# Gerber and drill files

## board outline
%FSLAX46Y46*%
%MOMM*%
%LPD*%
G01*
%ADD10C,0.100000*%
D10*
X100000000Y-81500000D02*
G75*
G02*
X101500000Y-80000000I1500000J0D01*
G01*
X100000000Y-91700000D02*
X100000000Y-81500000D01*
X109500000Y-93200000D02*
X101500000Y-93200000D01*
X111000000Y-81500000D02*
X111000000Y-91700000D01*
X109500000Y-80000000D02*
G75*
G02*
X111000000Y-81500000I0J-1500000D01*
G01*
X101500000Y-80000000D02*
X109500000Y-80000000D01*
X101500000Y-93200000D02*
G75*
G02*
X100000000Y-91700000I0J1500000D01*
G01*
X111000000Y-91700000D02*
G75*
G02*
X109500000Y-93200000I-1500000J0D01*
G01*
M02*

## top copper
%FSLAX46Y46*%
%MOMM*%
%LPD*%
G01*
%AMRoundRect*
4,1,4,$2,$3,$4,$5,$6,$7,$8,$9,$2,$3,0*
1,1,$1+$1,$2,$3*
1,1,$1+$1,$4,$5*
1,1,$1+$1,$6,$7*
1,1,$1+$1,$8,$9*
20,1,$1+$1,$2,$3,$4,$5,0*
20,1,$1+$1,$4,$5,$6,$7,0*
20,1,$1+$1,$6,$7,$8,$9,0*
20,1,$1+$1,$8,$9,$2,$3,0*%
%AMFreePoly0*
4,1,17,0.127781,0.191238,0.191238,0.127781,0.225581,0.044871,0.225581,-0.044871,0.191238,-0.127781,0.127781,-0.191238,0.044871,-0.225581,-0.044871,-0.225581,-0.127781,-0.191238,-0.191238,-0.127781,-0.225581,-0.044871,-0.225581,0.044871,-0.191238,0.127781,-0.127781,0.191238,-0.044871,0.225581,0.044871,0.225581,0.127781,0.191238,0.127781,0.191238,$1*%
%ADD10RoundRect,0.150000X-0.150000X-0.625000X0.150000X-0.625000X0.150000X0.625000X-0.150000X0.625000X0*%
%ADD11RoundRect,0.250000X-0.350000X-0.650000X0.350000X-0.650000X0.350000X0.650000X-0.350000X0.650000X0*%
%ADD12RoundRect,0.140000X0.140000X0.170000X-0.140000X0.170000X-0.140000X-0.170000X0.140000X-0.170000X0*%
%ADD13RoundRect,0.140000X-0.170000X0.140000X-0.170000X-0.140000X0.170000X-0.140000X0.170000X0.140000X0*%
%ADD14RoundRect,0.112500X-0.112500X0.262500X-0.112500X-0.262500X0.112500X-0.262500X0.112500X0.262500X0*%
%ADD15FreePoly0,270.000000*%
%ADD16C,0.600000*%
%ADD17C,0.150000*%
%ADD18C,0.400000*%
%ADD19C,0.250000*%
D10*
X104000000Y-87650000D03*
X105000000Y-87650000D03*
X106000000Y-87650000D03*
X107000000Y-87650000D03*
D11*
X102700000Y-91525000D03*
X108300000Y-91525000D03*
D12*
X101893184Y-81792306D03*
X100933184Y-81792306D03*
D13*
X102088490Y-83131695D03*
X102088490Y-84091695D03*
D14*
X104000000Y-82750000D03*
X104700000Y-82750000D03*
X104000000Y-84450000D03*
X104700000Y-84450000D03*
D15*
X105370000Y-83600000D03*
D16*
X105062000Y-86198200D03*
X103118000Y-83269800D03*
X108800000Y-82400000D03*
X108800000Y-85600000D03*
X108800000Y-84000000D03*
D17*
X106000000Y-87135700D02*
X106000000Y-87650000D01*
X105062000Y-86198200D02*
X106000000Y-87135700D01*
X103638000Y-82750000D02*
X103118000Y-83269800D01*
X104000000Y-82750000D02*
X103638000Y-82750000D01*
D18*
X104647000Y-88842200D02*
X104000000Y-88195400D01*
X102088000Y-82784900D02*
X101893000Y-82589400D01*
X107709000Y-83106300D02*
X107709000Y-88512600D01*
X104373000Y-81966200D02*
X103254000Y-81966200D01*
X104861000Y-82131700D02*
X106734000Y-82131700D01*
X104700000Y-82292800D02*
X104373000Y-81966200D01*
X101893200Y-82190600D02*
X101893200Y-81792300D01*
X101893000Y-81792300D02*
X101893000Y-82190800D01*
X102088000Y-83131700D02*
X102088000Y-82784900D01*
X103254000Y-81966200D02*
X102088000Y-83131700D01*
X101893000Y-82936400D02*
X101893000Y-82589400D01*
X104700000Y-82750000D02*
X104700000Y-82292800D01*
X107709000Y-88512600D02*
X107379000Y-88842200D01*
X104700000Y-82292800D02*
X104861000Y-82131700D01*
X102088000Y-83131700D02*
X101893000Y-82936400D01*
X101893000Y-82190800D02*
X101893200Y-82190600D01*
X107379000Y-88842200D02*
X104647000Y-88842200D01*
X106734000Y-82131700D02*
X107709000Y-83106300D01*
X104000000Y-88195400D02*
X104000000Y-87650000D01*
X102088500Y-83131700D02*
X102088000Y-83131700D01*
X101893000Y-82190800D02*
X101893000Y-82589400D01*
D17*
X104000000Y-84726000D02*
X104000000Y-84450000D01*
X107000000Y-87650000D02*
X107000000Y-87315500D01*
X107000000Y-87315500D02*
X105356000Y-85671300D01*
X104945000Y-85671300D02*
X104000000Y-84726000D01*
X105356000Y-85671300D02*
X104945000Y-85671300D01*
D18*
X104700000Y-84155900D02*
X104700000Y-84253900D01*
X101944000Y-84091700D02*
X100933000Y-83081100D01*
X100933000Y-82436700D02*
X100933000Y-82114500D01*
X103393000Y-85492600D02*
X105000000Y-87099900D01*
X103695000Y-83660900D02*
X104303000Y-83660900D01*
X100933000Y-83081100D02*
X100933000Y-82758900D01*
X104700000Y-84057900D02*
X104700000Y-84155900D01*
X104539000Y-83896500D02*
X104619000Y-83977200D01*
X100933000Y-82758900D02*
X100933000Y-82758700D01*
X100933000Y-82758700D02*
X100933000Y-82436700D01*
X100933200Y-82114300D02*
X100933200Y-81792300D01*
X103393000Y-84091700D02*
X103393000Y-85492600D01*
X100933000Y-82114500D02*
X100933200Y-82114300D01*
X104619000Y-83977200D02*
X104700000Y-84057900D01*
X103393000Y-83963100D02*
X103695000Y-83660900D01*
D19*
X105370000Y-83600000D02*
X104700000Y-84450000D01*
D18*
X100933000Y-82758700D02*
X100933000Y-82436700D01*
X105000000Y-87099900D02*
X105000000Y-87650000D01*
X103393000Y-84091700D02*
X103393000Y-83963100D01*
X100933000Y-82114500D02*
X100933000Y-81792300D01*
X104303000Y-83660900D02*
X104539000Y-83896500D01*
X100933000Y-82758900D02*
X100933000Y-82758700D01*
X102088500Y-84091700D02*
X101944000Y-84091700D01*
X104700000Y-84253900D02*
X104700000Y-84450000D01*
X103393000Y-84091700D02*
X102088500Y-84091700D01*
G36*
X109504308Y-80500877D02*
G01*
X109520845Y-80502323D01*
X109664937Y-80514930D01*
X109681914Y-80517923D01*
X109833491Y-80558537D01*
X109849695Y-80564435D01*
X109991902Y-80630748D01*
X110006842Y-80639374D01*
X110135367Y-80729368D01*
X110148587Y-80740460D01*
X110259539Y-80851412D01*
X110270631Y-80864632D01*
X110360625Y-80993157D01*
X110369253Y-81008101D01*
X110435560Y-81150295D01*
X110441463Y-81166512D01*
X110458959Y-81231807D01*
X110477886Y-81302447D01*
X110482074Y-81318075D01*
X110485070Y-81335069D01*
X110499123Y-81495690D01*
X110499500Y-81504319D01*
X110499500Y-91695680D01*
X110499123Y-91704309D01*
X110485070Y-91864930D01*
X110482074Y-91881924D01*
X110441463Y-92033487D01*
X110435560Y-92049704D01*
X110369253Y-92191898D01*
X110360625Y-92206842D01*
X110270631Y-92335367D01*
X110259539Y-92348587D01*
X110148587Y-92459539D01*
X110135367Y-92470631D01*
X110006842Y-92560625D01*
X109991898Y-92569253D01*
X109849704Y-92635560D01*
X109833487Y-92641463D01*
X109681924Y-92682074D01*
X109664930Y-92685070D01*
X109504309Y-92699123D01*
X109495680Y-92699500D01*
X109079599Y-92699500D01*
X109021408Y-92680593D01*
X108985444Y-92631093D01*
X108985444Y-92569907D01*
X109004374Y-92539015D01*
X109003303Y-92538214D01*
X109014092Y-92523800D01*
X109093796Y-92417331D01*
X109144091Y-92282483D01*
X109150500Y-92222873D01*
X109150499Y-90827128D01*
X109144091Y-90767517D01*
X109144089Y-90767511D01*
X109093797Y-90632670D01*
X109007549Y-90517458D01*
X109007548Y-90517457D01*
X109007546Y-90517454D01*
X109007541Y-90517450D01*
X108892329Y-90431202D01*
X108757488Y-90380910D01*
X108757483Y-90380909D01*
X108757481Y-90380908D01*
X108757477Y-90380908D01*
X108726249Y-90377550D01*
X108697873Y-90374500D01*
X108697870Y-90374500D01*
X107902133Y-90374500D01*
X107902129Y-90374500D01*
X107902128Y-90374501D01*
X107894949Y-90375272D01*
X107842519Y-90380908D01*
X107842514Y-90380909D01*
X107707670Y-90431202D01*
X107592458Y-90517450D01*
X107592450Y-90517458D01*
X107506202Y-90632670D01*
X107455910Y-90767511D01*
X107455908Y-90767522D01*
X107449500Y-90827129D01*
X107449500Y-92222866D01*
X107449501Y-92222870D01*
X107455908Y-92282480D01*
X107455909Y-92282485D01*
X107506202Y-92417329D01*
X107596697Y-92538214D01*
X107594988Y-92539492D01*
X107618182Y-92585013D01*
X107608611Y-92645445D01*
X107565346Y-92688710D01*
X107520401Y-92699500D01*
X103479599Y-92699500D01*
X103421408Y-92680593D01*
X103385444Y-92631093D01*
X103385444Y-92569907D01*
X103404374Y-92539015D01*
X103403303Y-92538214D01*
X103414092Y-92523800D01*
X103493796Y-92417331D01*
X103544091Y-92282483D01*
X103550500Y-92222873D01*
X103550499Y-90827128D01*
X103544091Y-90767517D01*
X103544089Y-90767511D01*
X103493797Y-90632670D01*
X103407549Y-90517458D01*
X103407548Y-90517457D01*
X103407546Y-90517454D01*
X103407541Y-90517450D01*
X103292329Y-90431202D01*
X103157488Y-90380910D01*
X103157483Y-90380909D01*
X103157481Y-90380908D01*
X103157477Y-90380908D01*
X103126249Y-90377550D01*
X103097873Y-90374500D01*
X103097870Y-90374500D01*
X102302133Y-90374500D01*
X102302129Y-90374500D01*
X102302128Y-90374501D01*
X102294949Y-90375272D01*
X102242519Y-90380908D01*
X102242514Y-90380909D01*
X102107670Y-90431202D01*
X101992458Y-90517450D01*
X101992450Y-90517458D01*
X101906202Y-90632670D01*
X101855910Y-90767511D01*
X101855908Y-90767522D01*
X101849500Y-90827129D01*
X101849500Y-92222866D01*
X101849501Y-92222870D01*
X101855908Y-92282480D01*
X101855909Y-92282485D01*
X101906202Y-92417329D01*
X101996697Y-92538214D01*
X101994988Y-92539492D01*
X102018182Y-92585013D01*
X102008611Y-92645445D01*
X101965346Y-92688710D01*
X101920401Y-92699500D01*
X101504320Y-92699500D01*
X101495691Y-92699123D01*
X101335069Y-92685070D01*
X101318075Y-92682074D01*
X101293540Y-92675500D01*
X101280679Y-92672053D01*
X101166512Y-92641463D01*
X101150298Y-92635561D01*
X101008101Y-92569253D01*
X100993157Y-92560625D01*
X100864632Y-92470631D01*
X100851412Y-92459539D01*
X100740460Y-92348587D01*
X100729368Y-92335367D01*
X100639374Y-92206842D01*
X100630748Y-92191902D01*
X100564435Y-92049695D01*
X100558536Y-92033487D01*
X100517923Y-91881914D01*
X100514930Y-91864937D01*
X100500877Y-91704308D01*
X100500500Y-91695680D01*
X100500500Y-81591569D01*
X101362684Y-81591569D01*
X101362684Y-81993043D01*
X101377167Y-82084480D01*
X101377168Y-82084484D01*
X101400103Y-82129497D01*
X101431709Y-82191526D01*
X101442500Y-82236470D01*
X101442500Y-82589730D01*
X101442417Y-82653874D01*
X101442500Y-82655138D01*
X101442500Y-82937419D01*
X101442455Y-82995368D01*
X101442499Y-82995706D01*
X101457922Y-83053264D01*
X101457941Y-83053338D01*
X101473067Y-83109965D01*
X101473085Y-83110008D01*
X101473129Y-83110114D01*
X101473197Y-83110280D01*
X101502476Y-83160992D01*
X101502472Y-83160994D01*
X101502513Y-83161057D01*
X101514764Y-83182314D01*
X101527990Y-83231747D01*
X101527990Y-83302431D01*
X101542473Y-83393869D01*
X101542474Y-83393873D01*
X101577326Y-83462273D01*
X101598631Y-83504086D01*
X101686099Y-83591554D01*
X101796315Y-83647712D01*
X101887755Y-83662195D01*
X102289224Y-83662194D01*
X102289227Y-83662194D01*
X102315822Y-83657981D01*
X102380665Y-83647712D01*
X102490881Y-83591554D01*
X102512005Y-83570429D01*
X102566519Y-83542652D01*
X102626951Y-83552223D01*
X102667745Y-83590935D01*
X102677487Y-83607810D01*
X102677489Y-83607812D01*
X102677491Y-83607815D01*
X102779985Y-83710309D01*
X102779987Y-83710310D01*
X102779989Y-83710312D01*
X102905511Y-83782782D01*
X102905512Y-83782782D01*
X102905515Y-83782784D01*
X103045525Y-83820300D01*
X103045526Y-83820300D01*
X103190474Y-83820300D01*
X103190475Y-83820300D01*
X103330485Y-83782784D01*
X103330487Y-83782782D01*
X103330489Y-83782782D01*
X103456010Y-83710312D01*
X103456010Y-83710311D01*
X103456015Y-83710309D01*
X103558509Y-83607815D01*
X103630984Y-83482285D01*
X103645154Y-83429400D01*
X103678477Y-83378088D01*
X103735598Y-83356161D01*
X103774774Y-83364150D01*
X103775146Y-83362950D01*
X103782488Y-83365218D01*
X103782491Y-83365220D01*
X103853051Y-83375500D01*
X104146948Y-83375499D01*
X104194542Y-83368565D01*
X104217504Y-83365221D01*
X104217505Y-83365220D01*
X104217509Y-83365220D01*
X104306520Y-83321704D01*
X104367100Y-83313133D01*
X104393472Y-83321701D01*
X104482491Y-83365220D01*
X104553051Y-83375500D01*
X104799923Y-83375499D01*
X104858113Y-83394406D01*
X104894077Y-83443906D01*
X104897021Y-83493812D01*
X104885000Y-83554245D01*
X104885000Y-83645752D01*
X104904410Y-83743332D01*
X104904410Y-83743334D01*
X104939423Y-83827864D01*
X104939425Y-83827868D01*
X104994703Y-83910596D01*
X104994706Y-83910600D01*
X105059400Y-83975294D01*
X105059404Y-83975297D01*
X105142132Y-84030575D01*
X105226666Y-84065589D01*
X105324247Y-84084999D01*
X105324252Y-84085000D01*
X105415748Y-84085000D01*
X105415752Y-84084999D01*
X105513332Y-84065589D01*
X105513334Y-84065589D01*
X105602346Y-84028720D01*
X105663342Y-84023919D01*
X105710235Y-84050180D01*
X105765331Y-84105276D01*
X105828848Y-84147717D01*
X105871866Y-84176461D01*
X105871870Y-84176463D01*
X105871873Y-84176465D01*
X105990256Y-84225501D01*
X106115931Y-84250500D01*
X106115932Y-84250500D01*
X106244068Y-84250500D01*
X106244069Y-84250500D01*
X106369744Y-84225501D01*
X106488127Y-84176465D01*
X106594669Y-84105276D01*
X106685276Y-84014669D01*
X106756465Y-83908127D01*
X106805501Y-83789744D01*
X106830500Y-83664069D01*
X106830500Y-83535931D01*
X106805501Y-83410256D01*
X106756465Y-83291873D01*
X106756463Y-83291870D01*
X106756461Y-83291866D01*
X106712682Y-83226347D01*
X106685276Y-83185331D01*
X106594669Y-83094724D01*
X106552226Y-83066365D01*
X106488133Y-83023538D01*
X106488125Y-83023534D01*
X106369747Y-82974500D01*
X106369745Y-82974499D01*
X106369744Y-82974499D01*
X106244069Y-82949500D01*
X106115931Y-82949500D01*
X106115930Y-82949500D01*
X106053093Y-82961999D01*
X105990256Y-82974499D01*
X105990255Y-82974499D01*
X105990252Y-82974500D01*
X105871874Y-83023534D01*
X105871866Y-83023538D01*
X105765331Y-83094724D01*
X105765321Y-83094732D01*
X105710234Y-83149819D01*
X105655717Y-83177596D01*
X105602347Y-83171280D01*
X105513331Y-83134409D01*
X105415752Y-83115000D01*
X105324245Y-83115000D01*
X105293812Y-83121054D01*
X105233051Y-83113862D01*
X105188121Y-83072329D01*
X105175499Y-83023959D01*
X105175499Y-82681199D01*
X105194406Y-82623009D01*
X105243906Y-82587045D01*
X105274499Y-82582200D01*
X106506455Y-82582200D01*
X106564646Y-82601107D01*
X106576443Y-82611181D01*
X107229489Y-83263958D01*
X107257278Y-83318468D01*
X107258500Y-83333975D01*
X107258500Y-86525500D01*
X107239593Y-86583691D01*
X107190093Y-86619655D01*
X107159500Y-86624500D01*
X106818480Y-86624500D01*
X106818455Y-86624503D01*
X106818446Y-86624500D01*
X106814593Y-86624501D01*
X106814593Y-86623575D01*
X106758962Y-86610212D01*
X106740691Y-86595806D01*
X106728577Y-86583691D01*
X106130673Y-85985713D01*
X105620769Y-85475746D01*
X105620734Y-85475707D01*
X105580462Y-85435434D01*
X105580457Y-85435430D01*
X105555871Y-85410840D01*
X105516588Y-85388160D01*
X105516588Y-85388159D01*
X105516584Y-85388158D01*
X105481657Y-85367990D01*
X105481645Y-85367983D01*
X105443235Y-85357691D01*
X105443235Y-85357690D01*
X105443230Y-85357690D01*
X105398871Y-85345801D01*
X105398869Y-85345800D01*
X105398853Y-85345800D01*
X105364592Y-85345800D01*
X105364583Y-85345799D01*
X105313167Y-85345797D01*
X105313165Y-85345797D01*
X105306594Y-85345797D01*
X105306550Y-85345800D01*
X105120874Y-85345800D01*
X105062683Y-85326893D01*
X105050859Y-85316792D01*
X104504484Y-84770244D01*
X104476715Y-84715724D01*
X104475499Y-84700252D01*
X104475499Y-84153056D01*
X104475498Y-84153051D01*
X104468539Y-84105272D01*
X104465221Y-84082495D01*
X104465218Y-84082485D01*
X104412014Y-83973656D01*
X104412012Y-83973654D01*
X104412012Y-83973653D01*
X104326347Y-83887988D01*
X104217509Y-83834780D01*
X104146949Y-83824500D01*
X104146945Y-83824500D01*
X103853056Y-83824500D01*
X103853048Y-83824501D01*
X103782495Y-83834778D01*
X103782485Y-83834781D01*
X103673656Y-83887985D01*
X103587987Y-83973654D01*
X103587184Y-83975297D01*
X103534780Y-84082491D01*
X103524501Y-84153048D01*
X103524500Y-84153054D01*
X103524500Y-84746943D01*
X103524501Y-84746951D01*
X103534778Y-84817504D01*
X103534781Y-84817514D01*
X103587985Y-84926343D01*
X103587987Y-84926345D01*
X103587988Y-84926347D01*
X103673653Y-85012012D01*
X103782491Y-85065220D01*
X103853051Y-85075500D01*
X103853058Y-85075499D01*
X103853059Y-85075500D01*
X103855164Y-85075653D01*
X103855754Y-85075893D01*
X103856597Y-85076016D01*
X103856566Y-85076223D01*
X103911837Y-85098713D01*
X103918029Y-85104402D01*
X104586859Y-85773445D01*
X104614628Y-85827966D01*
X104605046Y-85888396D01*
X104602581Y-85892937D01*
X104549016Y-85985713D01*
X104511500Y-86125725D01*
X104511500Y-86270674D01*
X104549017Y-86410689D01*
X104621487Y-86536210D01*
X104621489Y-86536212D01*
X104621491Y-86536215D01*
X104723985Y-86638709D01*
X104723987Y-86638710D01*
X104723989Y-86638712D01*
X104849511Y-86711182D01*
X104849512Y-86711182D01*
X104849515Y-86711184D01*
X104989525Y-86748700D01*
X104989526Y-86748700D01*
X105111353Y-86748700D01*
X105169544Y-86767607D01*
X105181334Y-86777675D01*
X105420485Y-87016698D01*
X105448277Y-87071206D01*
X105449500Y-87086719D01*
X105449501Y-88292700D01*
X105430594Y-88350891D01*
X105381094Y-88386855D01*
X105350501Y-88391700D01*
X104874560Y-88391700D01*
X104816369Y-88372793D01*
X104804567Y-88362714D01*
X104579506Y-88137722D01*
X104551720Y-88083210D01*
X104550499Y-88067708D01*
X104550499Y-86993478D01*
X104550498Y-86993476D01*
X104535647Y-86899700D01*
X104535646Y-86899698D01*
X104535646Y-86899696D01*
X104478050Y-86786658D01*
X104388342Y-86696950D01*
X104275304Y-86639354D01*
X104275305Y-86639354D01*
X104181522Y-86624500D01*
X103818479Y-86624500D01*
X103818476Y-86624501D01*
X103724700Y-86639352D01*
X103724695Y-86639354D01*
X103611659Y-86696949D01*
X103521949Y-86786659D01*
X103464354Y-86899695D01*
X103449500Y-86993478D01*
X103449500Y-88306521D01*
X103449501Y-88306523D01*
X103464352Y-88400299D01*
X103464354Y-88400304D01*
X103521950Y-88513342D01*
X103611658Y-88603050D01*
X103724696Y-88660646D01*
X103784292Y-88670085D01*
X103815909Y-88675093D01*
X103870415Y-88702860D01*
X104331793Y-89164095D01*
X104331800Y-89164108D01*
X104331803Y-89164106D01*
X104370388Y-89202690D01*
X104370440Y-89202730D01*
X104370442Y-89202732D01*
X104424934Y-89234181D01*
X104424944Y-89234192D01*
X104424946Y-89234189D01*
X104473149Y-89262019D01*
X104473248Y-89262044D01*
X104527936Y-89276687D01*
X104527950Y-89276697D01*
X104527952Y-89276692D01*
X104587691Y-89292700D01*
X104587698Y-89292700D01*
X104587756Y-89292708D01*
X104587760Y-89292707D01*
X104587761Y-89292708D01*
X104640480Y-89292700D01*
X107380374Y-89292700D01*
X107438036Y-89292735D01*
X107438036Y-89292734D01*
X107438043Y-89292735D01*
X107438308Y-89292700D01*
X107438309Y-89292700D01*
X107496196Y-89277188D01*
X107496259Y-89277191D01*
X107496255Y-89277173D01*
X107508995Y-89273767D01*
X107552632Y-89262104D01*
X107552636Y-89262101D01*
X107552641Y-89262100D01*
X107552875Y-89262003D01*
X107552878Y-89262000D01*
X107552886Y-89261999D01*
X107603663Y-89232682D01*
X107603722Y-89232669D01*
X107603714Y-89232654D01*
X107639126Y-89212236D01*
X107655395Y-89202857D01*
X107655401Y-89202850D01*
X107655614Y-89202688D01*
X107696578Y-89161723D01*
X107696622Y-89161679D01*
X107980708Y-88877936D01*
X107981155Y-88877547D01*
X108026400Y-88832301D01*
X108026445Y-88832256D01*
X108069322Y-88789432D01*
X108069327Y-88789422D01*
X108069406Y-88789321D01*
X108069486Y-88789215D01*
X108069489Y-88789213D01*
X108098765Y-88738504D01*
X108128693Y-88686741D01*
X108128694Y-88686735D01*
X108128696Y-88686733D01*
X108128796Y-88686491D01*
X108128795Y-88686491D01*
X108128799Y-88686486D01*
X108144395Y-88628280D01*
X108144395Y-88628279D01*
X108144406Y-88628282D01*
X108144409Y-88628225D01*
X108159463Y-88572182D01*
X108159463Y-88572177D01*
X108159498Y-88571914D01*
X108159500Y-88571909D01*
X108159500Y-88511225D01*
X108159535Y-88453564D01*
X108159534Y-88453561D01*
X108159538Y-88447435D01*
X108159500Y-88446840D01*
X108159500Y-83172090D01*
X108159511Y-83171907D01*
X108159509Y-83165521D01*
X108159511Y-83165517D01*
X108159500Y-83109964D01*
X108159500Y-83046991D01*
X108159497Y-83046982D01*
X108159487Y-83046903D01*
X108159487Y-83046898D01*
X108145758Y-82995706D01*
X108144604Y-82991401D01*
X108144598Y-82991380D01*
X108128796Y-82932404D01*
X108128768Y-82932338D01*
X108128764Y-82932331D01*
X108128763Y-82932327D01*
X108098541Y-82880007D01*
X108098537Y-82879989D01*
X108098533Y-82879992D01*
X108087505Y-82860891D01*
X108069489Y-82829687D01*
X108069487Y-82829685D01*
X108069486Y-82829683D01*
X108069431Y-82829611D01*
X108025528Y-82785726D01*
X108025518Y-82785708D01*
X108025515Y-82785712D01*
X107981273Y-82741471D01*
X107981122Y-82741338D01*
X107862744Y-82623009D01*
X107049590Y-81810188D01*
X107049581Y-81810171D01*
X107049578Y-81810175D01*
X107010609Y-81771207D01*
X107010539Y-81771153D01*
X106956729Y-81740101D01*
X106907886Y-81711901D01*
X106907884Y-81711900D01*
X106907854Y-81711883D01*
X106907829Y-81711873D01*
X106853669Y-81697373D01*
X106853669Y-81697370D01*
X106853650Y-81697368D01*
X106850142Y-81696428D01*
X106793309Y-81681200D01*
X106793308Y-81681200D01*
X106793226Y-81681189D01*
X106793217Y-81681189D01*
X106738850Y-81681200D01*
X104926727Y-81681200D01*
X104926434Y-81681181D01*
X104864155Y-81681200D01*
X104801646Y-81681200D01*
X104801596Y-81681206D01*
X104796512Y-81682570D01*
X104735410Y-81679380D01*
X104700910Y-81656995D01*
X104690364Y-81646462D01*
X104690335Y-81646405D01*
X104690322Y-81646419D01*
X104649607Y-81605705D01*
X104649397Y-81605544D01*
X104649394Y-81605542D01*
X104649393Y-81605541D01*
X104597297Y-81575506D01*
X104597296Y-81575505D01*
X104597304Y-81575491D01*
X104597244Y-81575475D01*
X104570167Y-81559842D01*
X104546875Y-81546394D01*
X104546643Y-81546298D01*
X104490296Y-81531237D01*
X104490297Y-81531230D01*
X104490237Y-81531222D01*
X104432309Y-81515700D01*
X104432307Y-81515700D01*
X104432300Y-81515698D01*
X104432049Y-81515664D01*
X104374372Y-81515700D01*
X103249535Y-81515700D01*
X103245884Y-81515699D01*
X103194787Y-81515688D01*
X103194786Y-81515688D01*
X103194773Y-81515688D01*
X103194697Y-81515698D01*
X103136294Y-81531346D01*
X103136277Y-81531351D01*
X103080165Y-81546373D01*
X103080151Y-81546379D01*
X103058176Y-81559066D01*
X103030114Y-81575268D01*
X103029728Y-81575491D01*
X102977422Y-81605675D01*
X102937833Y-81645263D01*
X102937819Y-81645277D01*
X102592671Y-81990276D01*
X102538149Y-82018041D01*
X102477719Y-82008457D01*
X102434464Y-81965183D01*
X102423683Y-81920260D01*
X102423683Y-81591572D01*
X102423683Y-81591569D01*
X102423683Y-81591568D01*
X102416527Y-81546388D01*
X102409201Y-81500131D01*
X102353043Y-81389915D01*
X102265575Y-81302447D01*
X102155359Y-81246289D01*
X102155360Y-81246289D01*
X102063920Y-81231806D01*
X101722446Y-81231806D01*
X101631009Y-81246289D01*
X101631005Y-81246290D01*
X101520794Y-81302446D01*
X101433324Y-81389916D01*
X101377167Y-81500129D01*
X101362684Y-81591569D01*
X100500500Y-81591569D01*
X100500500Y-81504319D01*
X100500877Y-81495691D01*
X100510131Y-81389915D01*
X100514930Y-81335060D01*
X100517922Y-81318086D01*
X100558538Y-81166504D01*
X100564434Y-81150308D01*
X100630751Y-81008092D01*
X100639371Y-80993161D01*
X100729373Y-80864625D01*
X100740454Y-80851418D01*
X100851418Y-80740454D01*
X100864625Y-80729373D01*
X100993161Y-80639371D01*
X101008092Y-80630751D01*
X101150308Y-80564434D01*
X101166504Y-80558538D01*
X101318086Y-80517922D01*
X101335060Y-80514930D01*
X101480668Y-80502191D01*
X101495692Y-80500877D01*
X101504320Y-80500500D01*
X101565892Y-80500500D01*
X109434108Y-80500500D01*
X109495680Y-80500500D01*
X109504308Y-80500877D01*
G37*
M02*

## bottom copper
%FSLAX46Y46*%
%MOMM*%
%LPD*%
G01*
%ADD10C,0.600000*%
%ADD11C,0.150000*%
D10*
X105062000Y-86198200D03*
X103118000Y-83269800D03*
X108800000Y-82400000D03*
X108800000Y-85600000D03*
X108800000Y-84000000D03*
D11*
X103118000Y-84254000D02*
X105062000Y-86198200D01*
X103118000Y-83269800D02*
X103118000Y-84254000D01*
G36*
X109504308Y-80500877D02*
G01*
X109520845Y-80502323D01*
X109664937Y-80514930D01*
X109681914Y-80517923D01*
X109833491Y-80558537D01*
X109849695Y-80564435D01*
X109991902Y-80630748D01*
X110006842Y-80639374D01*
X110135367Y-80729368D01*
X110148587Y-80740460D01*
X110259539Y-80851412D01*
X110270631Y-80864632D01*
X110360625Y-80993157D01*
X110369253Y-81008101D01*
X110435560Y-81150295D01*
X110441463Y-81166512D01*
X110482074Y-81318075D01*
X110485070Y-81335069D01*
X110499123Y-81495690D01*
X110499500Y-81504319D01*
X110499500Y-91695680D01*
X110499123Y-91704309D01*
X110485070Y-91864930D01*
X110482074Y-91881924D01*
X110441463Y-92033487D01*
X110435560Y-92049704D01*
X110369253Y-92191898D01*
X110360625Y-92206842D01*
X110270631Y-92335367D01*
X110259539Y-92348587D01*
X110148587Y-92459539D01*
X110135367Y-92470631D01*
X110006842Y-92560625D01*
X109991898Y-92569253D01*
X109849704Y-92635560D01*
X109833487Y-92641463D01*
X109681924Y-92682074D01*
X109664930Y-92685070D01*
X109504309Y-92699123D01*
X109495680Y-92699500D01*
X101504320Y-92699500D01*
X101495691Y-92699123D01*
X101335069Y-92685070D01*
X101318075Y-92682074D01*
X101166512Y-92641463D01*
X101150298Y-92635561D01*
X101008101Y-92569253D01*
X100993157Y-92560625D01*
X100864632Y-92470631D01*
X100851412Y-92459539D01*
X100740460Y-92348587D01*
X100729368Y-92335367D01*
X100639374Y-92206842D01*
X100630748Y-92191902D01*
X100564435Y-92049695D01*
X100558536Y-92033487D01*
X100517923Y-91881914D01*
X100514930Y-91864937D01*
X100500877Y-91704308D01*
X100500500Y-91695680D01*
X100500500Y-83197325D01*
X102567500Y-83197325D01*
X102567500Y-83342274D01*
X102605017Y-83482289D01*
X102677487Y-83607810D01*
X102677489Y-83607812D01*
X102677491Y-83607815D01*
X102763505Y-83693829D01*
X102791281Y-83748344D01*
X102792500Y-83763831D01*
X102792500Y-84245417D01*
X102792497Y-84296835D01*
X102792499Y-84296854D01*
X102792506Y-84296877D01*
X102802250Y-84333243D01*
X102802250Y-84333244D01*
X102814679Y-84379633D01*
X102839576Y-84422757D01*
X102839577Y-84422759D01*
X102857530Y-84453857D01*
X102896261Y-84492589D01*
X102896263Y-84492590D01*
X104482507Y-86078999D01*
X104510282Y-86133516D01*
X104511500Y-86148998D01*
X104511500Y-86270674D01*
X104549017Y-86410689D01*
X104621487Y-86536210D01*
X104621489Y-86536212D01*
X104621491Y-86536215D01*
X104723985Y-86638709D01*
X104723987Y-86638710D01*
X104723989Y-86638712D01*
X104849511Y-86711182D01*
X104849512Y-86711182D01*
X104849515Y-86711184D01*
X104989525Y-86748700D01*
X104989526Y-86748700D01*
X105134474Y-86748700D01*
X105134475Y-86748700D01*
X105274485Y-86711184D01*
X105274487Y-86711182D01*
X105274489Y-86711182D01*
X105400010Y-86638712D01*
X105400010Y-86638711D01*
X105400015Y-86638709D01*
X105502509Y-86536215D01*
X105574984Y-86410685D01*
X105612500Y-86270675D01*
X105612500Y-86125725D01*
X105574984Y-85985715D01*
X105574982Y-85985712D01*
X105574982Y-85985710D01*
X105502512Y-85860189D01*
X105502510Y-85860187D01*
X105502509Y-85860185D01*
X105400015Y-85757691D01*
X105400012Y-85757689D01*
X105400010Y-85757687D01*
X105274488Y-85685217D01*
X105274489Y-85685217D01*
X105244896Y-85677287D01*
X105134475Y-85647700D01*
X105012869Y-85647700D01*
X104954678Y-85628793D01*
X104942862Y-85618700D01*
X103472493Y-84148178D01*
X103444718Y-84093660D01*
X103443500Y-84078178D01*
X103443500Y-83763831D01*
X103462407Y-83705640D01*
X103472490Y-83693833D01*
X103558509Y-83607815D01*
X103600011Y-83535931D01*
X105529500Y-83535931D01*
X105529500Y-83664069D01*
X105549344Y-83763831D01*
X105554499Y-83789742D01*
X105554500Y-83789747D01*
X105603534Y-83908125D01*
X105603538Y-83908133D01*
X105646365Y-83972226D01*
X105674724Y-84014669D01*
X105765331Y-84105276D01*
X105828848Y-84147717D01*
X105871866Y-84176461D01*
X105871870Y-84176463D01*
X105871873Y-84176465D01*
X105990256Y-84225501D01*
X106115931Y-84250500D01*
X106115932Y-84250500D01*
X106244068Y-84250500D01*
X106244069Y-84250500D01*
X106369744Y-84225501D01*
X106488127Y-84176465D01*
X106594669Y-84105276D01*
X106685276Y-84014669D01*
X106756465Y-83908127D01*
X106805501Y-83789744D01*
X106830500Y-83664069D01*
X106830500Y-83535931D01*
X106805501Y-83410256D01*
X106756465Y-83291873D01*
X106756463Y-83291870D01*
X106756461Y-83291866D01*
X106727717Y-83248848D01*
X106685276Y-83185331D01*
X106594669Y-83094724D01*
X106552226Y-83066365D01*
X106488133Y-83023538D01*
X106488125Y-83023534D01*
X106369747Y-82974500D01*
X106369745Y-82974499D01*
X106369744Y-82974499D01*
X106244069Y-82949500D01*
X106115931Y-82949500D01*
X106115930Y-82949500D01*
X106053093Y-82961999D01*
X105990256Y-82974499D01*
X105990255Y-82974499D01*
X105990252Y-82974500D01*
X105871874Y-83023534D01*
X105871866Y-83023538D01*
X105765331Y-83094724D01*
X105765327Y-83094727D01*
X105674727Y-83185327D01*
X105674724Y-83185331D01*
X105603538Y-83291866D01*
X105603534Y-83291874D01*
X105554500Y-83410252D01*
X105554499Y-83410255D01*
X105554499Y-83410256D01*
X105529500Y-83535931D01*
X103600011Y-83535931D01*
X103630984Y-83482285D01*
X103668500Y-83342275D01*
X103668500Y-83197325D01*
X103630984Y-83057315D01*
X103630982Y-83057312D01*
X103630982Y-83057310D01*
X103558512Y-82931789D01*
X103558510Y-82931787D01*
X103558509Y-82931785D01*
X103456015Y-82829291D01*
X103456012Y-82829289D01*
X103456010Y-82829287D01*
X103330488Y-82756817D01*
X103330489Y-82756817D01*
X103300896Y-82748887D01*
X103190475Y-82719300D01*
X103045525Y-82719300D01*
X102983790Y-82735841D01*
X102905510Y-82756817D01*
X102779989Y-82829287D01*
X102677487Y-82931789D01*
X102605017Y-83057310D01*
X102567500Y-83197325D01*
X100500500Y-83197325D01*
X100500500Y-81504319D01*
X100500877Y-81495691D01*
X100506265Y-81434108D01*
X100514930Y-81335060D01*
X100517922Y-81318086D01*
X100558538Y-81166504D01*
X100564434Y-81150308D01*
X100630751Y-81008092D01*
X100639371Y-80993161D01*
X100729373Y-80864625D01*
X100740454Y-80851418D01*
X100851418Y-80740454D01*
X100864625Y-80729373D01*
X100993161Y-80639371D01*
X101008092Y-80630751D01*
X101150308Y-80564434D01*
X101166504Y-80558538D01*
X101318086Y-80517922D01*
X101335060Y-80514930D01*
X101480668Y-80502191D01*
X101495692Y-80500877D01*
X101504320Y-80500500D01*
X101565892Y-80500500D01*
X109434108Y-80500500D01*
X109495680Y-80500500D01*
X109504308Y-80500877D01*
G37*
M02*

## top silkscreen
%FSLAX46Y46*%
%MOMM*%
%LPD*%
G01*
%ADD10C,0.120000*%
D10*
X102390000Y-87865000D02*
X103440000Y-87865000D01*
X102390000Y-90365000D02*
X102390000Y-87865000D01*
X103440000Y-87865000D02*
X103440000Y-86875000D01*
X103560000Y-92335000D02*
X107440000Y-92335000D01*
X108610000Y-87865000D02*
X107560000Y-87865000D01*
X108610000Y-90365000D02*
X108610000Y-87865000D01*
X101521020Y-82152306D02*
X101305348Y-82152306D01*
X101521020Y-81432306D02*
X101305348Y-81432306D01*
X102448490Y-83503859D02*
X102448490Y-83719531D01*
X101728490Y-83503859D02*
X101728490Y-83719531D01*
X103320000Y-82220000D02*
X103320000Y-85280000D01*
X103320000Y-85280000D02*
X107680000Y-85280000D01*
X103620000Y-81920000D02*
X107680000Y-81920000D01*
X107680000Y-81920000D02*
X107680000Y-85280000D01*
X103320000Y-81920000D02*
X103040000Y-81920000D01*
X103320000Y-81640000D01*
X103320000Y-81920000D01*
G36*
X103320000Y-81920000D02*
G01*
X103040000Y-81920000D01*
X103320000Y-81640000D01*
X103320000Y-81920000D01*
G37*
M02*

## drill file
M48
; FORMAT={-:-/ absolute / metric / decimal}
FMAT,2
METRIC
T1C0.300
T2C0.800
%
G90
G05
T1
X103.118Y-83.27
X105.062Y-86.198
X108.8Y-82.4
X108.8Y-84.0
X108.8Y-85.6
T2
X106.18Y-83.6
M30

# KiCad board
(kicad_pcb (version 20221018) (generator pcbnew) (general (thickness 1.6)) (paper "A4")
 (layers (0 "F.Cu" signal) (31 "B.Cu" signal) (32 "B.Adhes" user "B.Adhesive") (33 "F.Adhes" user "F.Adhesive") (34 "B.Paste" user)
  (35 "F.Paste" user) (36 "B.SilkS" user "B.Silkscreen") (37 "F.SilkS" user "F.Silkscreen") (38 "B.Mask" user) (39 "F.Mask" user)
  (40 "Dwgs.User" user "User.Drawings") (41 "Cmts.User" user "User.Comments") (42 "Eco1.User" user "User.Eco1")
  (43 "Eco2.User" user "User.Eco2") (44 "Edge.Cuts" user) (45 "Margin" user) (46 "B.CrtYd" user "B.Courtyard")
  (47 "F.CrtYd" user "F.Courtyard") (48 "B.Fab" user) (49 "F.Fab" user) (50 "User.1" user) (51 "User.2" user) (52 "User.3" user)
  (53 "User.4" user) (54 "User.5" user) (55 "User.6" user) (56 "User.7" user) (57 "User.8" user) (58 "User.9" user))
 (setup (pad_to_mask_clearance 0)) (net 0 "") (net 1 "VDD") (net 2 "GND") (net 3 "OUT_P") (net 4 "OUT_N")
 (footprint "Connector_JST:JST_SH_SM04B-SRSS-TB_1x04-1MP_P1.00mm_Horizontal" (layer "F.Cu") (at 105.5 89.65) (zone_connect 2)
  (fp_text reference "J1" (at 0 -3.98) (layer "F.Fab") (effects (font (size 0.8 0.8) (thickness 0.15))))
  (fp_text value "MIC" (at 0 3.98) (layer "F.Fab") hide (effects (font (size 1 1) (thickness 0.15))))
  (fp_line (start -3.11 -1.785) (end -2.06 -1.785) (stroke (width 0.12) (type solid)) (layer "F.SilkS"))
  (fp_line (start -3.11 0.715) (end -3.11 -1.785) (stroke (width 0.12) (type solid)) (layer "F.SilkS"))
  (fp_line (start -2.06 -1.785) (end -2.06 -2.775) (stroke (width 0.12) (type solid)) (layer "F.SilkS"))
  (fp_line (start -1.94 2.685) (end 1.94 2.685) (stroke (width 0.12) (type solid)) (layer "F.SilkS"))
  (fp_line (start 3.11 -1.785) (end 2.06 -1.785) (stroke (width 0.12) (type solid)) (layer "F.SilkS"))
  (fp_line (start 3.11 0.715) (end 3.11 -1.785) (stroke (width 0.12) (type solid)) (layer "F.SilkS"))
  (pad "1" smd roundrect (at -1.5 -2) (size 0.6 1.55) (layers "F.Cu" "F.Paste" "F.Mask") (roundrect_rratio 0.25) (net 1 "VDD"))
  (pad "2" smd roundrect (at -0.5 -2) (size 0.6 1.55) (layers "F.Cu" "F.Paste" "F.Mask") (roundrect_rratio 0.25) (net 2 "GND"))
  (pad "3" smd roundrect (at 0.5 -2) (size 0.6 1.55) (layers "F.Cu" "F.Paste" "F.Mask") (roundrect_rratio 0.25) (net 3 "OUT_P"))
  (pad "4" smd roundrect (at 1.5 -2) (size 0.6 1.55) (layers "F.Cu" "F.Paste" "F.Mask") (roundrect_rratio 0.25) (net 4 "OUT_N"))
  (pad "MP" smd roundrect (at -2.8 1.875) (size 1.2 1.8) (layers "F.Cu" "F.Paste" "F.Mask") (roundrect_rratio 0.208333))
  (pad "MP" smd roundrect (at 2.8 1.875) (size 1.2 1.8) (layers "F.Cu" "F.Paste" "F.Mask") (roundrect_rratio 0.208333)))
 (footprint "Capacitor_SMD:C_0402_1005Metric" (layer "F.Cu") (at 101.413184 81.792306 180) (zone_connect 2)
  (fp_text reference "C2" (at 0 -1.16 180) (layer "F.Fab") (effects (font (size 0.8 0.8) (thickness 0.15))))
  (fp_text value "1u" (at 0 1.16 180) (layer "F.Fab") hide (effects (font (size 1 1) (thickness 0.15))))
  (fp_line (start -0.107836 -0.36) (end 0.107836 -0.36) (stroke (width 0.12) (type solid)) (layer "F.SilkS"))
  (fp_line (start -0.107836 0.36) (end 0.107836 0.36) (stroke (width 0.12) (type solid)) (layer "F.SilkS"))
  (pad "1" smd roundrect (at -0.48 0 180) (size 0.56 0.62) (layers "F.Cu" "F.Paste" "F.Mask") (roundrect_rratio 0.25) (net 1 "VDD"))
  (pad "2" smd roundrect (at 0.48 0 180) (size 0.56 0.62) (layers "F.Cu" "F.Paste" "F.Mask") (roundrect_rratio 0.25) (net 2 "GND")))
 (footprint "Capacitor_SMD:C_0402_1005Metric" (layer "F.Cu") (at 102.08849 83.611695 -90) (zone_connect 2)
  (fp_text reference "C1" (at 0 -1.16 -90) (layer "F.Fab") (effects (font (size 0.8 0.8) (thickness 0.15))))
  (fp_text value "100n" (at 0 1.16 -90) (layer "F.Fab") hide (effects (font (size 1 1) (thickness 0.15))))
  (fp_line (start -0.107836 -0.36) (end 0.107836 -0.36) (stroke (width 0.12) (type solid)) (layer "F.SilkS"))
  (fp_line (start -0.107836 0.36) (end 0.107836 0.36) (stroke (width 0.12) (type solid)) (layer "F.SilkS"))
  (pad "1" smd roundrect (at -0.48 0 270) (size 0.56 0.62) (layers "F.Cu" "F.Paste" "F.Mask") (roundrect_rratio 0.25) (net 1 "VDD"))
  (pad "2" smd roundrect (at 0.48 0 270) (size 0.56 0.62) (layers "F.Cu" "F.Paste" "F.Mask") (roundrect_rratio 0.25) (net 2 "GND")))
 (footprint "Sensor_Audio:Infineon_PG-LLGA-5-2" (layer "F.Cu") (at 105.5 83.6) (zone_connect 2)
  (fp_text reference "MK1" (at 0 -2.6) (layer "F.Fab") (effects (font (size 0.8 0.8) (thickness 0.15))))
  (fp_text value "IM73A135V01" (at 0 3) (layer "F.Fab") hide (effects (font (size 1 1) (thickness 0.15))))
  (fp_line (start -2.18 -1.38) (end -2.18 1.68) (stroke (width 0.12) (type solid)) (layer "F.SilkS"))
  (fp_line (start -2.18 1.68) (end 2.18 1.68) (stroke (width 0.12) (type solid)) (layer "F.SilkS"))
  (fp_line (start -1.88 -1.68) (end 2.18 -1.68) (stroke (width 0.12) (type solid)) (layer "F.SilkS"))
  (fp_line (start 2.18 -1.68) (end 2.18 1.68) (stroke (width 0.12) (type solid)) (layer "F.SilkS"))
  (fp_poly
   (pts (xy -2.18 -1.68) (xy -2.46 -1.68) (xy -2.18 -1.96) (xy -2.18 -1.68)) (stroke (width 0.12) (type solid)) (fill solid)
   (layer "F.SilkS"))
  (pad "" np_thru_hole circle (at 0.68 0 90) (size 0.8 0.8) (drill 0.8) (layers "F&B.Cu" "*.Mask"))
  (pad "1" smd roundrect (at -1.5 -0.85 270) (size 0.75 0.45) (layers "F.Cu" "F.Mask") (roundrect_rratio 0.25) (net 3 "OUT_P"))
  (pad "2" smd roundrect (at -0.8 -0.85 270) (size 0.75 0.45) (layers "F.Cu" "F.Mask") (roundrect_rratio 0.25) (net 1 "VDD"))
  (pad "3" smd roundrect (at -1.5 0.85 270) (size 0.75 0.45) (layers "F.Cu" "F.Mask") (roundrect_rratio 0.25) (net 4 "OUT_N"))
  (pad "4" smd roundrect (at -0.8 0.85 270) (size 0.75 0.45) (layers "F.Cu" "F.Mask") (roundrect_rratio 0.25) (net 2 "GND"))
  (pad "5" smd custom (at -0.13 0 270) (size 0.46 0.46) (layers "F.Cu" "F.Mask") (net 2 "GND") (zone_connect 0)
   (options (clearance outline) (anchor circle)) (primitives)))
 (gr_arc (start 100 81.5) (mid 100.43934 80.43934) (end 101.5 80) (stroke (width 0.1) (type default)) (layer "Edge.Cuts"))
 (gr_line (start 100 91.7) (end 100 81.5) (stroke (width 0.1) (type default)) (layer "Edge.Cuts"))
 (gr_line (start 109.5 93.2) (end 101.5 93.2) (stroke (width 0.1) (type default)) (layer "Edge.Cuts"))
 (gr_line (start 111 81.5) (end 111 91.7) (stroke (width 0.1) (type default)) (layer "Edge.Cuts"))
 (gr_arc (start 109.5 80) (mid 110.56066 80.43934) (end 111 81.5) (stroke (width 0.1) (type default)) (layer "Edge.Cuts"))
 (gr_line (start 101.5 80) (end 109.5 80) (stroke (width 0.1) (type default)) (layer "Edge.Cuts"))
 (gr_arc (start 101.5 93.2) (mid 100.43934 92.76066) (end 100 91.7) (stroke (width 0.1) (type default)) (layer "Edge.Cuts"))
 (gr_arc (start 111 91.7) (mid 110.56066 92.76066) (end 109.5 93.2) (stroke (width 0.1) (type default)) (layer "Edge.Cuts"))
 (segment (start 106 87.1357) (end 106 87.65) (width 0.15) (layer "F.Cu") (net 3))
 (segment (start 105.062 86.1982) (end 106 87.1357) (width 0.15) (layer "F.Cu") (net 3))
 (segment (start 103.638 82.75) (end 103.118 83.2698) (width 0.15) (layer "F.Cu") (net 3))
 (segment (start 104 82.75) (end 103.638 82.75) (width 0.15) (layer "F.Cu") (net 3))
 (via (at 105.062 86.1982) (size 0.6) (drill 0.3) (layers "F.Cu" "B.Cu") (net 3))
 (via (at 103.118 83.2698) (size 0.6) (drill 0.3) (layers "F.Cu" "B.Cu") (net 3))
 (segment (start 103.118 84.254) (end 105.062 86.1982) (width 0.15) (layer "B.Cu") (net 3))
 (segment (start 103.118 83.2698) (end 103.118 84.254) (width 0.15) (layer "B.Cu") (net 3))
 (segment (start 104.647 88.8422) (end 104 88.1954) (width 0.4) (layer "F.Cu") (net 1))
 (segment (start 102.088 82.7849) (end 101.893 82.5894) (width 0.4) (layer "F.Cu") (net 1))
 (segment (start 107.709 83.1063) (end 107.709 88.5126) (width 0.4) (layer "F.Cu") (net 1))
 (segment (start 104.373 81.9662) (end 103.254 81.9662) (width 0.4) (layer "F.Cu") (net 1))
 (segment (start 104.861 82.1317) (end 106.734 82.1317) (width 0.4) (layer "F.Cu") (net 1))
 (segment (start 104.7 82.2928) (end 104.373 81.9662) (width 0.4) (layer "F.Cu") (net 1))
 (segment (start 101.8932 82.1906) (end 101.8932 81.7923) (width 0.4) (layer "F.Cu") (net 1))
 (segment (start 101.893 81.7923) (end 101.893 82.1908) (width 0.4) (layer "F.Cu") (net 1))
 (segment (start 102.088 83.1317) (end 102.088 82.7849) (width 0.4) (layer "F.Cu") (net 1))
 (segment (start 103.254 81.9662) (end 102.088 83.1317) (width 0.4) (layer "F.Cu") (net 1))
 (segment (start 101.893 82.9364) (end 101.893 82.5894) (width 0.4) (layer "F.Cu") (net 1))
 (segment (start 104.7 82.75) (end 104.7 82.2928) (width 0.4) (layer "F.Cu") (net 1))
 (segment (start 107.709 88.5126) (end 107.379 88.8422) (width 0.4) (layer "F.Cu") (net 1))
 (segment (start 104.7 82.2928) (end 104.861 82.1317) (width 0.4) (layer "F.Cu") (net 1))
 (segment (start 102.088 83.1317) (end 101.893 82.9364) (width 0.4) (layer "F.Cu") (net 1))
 (segment (start 101.893 82.1908) (end 101.8932 82.1906) (width 0.4) (layer "F.Cu") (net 1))
 (segment (start 107.379 88.8422) (end 104.647 88.8422) (width 0.4) (layer "F.Cu") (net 1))
 (segment (start 106.734 82.1317) (end 107.709 83.1063) (width 0.4) (layer "F.Cu") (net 1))
 (segment (start 104 88.1954) (end 104 87.65) (width 0.4) (layer "F.Cu") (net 1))
 (segment (start 102.0885 83.1317) (end 102.088 83.1317) (width 0.4) (layer "F.Cu") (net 1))
 (segment (start 101.893 82.1908) (end 101.893 82.5894) (width 0.4) (layer "F.Cu") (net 1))
 (segment (start 104 84.726) (end 104 84.45) (width 0.15) (layer "F.Cu") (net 4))
 (segment (start 107 87.65) (end 107 87.3155) (width 0.15) (layer "F.Cu") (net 4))
 (segment (start 107 87.3155) (end 105.356 85.6713) (width 0.15) (layer "F.Cu") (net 4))
 (segment (start 104.945 85.6713) (end 104 84.726) (width 0.15) (layer "F.Cu") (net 4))
 (segment (start 105.356 85.6713) (end 104.945 85.6713) (width 0.15) (layer "F.Cu") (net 4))
 (segment (start 104.7 84.1559) (end 104.7 84.2539) (width 0.4) (layer "F.Cu") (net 2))
 (segment (start 101.944 84.0917) (end 100.933 83.0811) (width 0.4) (layer "F.Cu") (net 2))
 (segment (start 100.933 82.4367) (end 100.933 82.1145) (width 0.4) (layer "F.Cu") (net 2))
 (segment (start 103.393 85.4926) (end 105 87.0999) (width 0.4) (layer "F.Cu") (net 2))
 (segment (start 103.695 83.6609) (end 104.303 83.6609) (width 0.4) (layer "F.Cu") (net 2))
 (segment (start 100.933 83.0811) (end 100.933 82.7589) (width 0.4) (layer "F.Cu") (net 2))
 (segment (start 104.7 84.0579) (end 104.7 84.1559) (width 0.4) (layer "F.Cu") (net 2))
 (segment (start 104.539 83.8965) (end 104.619 83.9772) (width 0.4) (layer "F.Cu") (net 2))
 (segment (start 100.933 82.7589) (end 100.933 82.7587) (width 0.4) (layer "F.Cu") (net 2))
 (segment (start 100.933 82.7587) (end 100.933 82.4367) (width 0.4) (layer "F.Cu") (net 2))
 (segment (start 100.9332 82.1143) (end 100.9332 81.7923) (width 0.4) (layer "F.Cu") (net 2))
 (segment (start 103.393 84.0917) (end 103.393 85.4926) (width 0.4) (layer "F.Cu") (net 2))
 (segment (start 100.933 82.1145) (end 100.9332 82.1143) (width 0.4) (layer "F.Cu") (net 2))
 (segment (start 104.619 83.9772) (end 104.7 84.0579) (width 0.4) (layer "F.Cu") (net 2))
 (segment (start 103.393 83.9631) (end 103.695 83.6609) (width 0.4) (layer "F.Cu") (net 2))
 (segment (start 105.37 83.6) (end 104.7 84.45) (width 0.25) (layer "F.Cu") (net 2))
 (segment (start 100.933 82.7587) (end 100.933 82.4367) (width 0.4) (layer "F.Cu") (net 2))
 (segment (start 105 87.0999) (end 105 87.65) (width 0.4) (layer "F.Cu") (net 2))
 (segment (start 103.393 84.0917) (end 103.393 83.9631) (width 0.4) (layer "F.Cu") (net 2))
 (segment (start 100.933 82.1145) (end 100.933 81.7923) (width 0.4) (layer "F.Cu") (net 2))
 (segment (start 104.303 83.6609) (end 104.539 83.8965) (width 0.4) (layer "F.Cu") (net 2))
 (segment (start 100.933 82.7589) (end 100.933 82.7587) (width 0.4) (layer "F.Cu") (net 2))
 (segment (start 102.0885 84.0917) (end 101.944 84.0917) (width 0.4) (layer "F.Cu") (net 2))
 (segment (start 104.7 84.2539) (end 104.7 84.45) (width 0.4) (layer "F.Cu") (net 2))
 (segment (start 103.393 84.0917) (end 102.0885 84.0917) (width 0.4) (layer "F.Cu") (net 2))
 (via (at 108.8 82.4) (size 0.6) (drill 0.3) (layers "F.Cu" "B.Cu") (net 2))
 (via (at 108.8 85.6) (size 0.6) (drill 0.3) (layers "F.Cu" "B.Cu") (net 2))
 (via (at 108.8 84) (size 0.6) (drill 0.3) (layers "F.Cu" "B.Cu") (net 2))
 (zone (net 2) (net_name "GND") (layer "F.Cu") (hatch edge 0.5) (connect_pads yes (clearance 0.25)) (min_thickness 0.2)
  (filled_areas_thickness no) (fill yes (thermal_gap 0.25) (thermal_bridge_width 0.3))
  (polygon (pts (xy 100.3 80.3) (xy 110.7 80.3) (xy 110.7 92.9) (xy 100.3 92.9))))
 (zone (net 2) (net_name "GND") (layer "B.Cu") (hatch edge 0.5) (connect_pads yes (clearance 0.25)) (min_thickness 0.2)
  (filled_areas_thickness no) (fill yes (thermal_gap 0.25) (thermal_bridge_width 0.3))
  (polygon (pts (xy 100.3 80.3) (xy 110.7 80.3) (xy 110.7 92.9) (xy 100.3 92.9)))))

